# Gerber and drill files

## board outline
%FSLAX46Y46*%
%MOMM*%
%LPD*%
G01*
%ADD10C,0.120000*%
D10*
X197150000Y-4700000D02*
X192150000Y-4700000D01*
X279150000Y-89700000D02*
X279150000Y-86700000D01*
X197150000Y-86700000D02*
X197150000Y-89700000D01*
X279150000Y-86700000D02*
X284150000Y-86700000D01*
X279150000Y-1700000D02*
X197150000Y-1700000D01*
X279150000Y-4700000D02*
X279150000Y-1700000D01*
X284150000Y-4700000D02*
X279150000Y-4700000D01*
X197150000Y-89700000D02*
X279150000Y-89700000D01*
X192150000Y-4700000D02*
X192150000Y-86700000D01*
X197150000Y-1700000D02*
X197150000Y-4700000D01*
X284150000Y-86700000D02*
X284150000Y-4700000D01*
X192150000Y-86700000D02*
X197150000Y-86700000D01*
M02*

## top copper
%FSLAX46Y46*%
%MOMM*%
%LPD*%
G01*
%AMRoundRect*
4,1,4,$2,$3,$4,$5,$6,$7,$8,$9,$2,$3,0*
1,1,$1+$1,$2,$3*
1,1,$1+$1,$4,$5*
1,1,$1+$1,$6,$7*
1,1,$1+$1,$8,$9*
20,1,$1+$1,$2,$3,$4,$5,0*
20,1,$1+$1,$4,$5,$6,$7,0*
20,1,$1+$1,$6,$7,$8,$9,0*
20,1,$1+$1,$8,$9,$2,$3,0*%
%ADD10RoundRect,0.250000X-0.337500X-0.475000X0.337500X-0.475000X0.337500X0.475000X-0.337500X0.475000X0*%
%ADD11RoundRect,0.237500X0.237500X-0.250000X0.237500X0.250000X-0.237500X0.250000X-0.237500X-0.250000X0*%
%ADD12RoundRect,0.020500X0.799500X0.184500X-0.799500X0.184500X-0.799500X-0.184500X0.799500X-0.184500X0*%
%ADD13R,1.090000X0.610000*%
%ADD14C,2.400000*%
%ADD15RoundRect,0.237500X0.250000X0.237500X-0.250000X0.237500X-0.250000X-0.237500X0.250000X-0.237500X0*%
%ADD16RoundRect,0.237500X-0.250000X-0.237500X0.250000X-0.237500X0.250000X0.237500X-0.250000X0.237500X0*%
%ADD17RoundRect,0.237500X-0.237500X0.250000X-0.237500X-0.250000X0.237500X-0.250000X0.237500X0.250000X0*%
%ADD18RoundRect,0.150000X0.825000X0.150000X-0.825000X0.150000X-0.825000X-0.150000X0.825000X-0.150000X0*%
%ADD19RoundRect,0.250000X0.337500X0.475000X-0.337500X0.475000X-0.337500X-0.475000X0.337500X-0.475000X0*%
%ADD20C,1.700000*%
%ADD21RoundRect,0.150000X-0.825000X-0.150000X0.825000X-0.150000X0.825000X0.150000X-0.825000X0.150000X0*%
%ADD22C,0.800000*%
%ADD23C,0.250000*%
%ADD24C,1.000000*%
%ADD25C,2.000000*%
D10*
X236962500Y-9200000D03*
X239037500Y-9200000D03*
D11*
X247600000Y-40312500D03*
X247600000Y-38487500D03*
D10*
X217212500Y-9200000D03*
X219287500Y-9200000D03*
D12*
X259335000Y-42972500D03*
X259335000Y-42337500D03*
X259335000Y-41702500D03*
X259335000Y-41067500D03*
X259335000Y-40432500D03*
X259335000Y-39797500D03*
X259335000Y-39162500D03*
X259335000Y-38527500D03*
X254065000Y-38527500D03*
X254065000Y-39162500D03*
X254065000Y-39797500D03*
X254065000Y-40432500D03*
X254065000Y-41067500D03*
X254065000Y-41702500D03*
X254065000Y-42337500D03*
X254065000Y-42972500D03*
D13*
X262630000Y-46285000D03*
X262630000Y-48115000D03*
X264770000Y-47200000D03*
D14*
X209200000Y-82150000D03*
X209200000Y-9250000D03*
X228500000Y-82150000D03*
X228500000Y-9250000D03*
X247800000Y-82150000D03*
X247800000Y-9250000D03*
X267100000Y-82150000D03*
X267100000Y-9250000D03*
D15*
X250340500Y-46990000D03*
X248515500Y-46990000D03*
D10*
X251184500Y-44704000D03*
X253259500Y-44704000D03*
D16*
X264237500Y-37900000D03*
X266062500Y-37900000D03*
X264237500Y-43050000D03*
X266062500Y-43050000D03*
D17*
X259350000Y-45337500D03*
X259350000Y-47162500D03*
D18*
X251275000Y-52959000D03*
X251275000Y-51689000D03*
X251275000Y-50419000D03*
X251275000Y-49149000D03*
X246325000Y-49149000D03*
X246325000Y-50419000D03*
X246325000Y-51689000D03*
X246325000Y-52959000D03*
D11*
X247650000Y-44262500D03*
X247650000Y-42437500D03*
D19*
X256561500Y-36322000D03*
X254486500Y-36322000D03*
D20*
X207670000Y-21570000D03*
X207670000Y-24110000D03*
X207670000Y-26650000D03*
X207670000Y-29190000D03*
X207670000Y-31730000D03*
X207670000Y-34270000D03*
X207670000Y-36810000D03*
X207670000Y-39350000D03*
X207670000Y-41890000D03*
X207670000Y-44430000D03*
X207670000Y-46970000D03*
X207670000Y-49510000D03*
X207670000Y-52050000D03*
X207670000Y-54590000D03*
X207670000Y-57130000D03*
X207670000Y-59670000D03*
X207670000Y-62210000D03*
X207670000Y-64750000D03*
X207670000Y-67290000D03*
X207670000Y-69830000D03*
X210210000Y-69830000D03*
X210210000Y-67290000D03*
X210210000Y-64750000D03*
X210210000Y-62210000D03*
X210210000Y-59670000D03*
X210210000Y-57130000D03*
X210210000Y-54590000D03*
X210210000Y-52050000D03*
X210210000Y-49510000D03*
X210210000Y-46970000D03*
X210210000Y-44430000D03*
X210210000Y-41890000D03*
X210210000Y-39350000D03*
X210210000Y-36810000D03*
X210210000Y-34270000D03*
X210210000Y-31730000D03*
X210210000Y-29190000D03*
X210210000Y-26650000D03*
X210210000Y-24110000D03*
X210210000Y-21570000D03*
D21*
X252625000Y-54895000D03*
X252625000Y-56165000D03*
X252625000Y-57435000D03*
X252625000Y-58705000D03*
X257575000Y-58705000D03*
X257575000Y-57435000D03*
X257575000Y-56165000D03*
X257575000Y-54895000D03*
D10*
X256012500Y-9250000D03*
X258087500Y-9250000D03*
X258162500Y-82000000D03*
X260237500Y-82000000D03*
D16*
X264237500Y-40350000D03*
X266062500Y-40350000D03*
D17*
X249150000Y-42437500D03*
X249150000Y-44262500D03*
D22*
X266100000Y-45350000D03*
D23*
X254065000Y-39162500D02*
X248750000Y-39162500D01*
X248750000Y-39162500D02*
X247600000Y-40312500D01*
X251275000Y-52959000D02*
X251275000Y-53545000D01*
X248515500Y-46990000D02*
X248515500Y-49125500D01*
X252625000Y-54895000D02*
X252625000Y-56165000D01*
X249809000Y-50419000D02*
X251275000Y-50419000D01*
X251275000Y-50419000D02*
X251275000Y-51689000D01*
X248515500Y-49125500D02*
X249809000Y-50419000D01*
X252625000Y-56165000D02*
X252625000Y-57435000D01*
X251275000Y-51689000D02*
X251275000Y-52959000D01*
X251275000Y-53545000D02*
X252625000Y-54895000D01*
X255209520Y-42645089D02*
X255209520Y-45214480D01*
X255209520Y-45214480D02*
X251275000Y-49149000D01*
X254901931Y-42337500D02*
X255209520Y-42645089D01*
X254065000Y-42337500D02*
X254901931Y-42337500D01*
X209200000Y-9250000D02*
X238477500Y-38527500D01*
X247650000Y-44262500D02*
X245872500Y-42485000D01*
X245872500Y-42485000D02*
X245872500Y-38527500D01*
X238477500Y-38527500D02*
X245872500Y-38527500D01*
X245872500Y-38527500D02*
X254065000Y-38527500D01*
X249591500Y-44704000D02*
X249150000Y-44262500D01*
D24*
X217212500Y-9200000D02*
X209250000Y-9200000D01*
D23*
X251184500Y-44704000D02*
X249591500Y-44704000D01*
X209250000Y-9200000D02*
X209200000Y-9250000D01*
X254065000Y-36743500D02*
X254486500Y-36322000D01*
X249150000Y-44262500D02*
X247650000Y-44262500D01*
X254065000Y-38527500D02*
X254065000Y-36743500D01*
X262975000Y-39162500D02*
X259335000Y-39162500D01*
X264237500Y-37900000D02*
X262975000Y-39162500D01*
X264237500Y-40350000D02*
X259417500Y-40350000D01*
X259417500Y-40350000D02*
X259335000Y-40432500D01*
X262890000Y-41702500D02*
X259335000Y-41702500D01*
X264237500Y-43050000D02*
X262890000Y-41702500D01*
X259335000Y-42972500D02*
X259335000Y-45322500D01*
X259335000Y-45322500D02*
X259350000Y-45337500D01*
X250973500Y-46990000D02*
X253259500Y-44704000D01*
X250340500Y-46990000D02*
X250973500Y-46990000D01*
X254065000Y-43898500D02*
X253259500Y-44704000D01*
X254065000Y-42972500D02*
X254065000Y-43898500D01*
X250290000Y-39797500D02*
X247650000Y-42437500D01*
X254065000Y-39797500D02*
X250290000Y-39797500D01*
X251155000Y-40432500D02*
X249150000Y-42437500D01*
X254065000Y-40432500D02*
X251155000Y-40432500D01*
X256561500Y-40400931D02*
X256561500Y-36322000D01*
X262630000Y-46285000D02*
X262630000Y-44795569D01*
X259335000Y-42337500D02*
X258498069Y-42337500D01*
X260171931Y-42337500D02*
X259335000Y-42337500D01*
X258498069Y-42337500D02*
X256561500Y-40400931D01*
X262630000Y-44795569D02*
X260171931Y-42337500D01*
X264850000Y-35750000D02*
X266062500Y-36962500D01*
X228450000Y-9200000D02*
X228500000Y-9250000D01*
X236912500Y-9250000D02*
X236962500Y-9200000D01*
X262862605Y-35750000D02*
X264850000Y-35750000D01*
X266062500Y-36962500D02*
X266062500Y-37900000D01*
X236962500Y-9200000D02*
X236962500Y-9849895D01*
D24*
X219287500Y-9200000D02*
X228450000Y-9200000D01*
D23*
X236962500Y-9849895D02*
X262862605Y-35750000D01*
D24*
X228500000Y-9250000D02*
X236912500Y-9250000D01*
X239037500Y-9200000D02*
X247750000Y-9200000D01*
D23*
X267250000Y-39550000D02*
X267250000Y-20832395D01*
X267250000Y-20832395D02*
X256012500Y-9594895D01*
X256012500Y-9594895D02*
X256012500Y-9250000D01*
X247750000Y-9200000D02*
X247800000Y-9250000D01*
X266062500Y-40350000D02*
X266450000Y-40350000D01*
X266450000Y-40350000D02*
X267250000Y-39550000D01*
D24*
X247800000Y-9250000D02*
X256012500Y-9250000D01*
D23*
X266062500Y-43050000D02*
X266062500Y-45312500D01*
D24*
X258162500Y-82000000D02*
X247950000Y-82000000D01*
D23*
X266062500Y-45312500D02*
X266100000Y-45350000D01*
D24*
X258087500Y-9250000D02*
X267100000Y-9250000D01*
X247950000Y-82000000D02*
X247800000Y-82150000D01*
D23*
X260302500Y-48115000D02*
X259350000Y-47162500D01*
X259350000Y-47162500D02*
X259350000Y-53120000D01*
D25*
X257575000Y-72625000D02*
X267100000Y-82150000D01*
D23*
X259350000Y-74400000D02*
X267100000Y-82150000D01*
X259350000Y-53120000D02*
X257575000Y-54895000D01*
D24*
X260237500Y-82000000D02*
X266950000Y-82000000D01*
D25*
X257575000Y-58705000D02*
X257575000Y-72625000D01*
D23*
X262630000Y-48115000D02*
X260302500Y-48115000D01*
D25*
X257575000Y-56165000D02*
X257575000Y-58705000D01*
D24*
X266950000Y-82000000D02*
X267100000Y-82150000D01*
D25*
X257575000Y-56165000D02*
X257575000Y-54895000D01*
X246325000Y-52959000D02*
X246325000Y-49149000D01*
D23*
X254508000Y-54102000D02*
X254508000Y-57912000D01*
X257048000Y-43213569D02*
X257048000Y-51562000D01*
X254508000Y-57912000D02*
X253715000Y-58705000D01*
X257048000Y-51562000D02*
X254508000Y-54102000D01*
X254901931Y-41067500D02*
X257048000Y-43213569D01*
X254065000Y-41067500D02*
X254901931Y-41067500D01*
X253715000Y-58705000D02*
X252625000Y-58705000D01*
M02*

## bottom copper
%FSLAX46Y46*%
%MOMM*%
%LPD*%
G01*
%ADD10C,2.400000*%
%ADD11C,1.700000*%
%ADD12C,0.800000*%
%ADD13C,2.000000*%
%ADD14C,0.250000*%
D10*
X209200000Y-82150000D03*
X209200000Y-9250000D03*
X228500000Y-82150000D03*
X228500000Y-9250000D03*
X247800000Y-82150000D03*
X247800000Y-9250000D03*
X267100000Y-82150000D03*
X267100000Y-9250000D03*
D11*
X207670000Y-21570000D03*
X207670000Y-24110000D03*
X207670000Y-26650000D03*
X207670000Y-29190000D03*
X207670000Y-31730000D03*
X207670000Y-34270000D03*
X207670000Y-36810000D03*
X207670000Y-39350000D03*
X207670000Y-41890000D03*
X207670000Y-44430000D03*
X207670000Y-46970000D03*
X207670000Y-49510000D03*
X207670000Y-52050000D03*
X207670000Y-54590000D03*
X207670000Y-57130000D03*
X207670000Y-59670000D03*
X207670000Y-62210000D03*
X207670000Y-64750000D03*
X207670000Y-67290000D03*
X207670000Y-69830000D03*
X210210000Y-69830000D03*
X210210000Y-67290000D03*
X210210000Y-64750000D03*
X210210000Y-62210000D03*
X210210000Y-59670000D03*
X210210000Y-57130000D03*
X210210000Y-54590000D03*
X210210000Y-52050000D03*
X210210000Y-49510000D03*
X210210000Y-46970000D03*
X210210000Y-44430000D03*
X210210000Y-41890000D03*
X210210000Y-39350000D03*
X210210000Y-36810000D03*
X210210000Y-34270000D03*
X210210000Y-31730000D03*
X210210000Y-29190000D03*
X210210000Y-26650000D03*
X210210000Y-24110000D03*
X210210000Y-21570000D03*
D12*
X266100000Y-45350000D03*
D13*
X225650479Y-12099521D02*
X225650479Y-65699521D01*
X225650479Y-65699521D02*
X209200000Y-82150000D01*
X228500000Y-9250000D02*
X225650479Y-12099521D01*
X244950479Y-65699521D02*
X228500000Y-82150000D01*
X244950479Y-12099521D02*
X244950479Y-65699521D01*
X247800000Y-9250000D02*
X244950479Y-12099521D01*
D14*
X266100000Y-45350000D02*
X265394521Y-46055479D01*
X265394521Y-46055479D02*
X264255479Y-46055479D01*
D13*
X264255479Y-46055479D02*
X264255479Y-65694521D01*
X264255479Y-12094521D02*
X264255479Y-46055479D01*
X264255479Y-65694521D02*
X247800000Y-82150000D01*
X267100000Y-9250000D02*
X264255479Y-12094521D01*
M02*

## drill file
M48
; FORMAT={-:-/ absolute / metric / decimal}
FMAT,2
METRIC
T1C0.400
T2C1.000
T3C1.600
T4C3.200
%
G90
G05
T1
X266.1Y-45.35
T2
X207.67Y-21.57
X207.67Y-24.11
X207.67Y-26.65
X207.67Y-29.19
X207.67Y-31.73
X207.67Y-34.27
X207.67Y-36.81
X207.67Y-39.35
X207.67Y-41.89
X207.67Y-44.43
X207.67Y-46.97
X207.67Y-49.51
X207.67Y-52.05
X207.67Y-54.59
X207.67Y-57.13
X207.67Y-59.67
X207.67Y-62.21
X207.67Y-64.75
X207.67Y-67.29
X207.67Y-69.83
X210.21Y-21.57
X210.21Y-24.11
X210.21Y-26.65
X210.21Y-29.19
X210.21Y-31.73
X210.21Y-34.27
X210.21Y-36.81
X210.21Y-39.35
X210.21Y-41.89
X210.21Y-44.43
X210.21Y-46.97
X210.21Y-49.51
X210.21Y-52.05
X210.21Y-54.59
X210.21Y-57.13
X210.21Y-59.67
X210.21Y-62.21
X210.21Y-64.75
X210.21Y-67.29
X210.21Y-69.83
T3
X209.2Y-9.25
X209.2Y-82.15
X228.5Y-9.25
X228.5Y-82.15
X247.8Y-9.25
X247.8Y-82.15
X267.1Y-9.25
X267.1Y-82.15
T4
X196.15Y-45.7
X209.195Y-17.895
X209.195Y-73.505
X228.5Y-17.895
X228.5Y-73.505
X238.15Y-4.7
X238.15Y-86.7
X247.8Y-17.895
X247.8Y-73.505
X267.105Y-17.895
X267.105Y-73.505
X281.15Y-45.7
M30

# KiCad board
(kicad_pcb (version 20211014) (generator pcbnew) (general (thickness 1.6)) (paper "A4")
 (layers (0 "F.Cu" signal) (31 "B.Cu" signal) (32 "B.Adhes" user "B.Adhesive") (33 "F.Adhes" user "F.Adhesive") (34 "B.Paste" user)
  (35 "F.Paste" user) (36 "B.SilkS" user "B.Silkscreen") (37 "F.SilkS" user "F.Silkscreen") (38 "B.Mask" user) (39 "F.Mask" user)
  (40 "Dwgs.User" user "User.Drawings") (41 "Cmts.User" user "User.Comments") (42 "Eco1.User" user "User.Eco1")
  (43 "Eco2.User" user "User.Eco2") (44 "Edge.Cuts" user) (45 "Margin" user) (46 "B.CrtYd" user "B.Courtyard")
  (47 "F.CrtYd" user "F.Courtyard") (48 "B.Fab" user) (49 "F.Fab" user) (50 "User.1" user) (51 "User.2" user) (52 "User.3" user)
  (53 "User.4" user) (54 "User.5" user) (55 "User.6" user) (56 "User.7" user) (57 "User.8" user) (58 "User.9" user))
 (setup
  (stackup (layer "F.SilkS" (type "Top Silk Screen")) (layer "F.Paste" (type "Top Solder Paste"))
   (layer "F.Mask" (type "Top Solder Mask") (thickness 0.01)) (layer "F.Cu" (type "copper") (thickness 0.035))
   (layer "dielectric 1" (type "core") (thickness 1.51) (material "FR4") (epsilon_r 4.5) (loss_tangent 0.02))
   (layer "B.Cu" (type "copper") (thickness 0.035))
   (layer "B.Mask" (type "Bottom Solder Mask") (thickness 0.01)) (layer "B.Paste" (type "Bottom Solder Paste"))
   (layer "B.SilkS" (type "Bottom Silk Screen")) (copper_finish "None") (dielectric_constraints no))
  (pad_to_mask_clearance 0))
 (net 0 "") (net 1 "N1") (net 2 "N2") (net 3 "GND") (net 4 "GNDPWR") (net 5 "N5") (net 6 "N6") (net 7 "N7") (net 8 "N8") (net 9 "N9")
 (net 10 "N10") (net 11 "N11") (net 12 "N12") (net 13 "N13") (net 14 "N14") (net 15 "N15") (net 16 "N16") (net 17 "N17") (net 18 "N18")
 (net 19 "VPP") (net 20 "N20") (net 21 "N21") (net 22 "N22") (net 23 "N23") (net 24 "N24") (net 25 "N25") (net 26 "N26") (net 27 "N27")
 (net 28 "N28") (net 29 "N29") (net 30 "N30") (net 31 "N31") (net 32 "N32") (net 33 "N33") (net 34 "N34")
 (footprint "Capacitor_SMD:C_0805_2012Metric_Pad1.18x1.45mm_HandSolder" (layer "F.Cu") (at 238 9.2)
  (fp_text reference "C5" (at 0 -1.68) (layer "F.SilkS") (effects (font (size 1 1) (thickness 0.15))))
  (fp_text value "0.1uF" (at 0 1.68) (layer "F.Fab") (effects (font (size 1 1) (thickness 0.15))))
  (pad "1" smd roundrect (at -1.0375 0) (size 1.175 1.45) (layers "F.Cu" "F.Paste" "F.Mask") (roundrect_rratio 0.212766) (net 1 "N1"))
  (pad "2" smd roundrect (at 1.0375 0) (size 1.175 1.45) (layers "F.Cu" "F.Paste" "F.Mask") (roundrect_rratio 0.212766) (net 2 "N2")))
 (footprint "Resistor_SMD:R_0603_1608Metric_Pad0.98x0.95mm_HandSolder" (layer "F.Cu") (at 247.6 39.4 90)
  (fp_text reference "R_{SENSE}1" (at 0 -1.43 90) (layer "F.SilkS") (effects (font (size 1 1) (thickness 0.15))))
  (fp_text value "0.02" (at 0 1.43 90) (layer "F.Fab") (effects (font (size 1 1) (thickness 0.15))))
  (pad "1" smd roundrect (at -0.9125 0 90) (size 0.975 0.95) (layers "F.Cu" "F.Paste" "F.Mask") (roundrect_rratio 0.25) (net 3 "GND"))
  (pad "2" smd roundrect (at 0.9125 0 90) (size 0.975 0.95) (layers "F.Cu" "F.Paste" "F.Mask") (roundrect_rratio 0.25) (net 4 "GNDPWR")))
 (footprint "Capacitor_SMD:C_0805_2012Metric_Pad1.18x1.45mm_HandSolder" (layer "F.Cu") (at 218.25 9.2)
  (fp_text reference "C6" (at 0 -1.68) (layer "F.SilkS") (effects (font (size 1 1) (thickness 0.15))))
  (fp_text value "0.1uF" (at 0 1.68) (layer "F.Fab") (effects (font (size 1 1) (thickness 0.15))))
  (pad "1" smd roundrect (at -1.0375 0) (size 1.175 1.45) (layers "F.Cu" "F.Paste" "F.Mask") (roundrect_rratio 0.212766) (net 4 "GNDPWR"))
  (pad "2" smd roundrect (at 1.0375 0) (size 1.175 1.45) (layers "F.Cu" "F.Paste" "F.Mask") (roundrect_rratio 0.212766) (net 1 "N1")))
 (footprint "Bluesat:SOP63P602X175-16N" (layer "F.Cu") (at 256.7 40.75 180)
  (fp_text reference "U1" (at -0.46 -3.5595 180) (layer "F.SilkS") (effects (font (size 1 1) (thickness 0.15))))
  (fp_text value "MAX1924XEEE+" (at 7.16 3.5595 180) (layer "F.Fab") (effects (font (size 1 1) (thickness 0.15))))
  (pad "1" smd roundrect locked (at -2.635 -2.2225 180) (size 1.64 0.41) (layers "F.Cu" "F.Paste" "F.Mask") (roundrect_rratio 0.05)
   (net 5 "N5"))
  (pad "2" smd roundrect locked (at -2.635 -1.5875 180) (size 1.64 0.41) (layers "F.Cu" "F.Paste" "F.Mask") (roundrect_rratio 0.05)
   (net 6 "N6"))
  (pad "3" smd roundrect locked (at -2.635 -0.9525 180) (size 1.64 0.41) (layers "F.Cu" "F.Paste" "F.Mask") (roundrect_rratio 0.05)
   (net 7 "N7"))
  (pad "4" smd roundrect locked (at -2.635 -0.3175 180) (size 1.64 0.41) (layers "F.Cu" "F.Paste" "F.Mask") (roundrect_rratio 0.05))
  (pad "5" smd roundrect locked (at -2.635 0.3175 180) (size 1.64 0.41) (layers "F.Cu" "F.Paste" "F.Mask") (roundrect_rratio 0.05)
   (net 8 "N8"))
  (pad "6" smd roundrect locked (at -2.635 0.9525 180) (size 1.64 0.41) (layers "F.Cu" "F.Paste" "F.Mask") (roundrect_rratio 0.05))
  (pad "7" smd roundrect locked (at -2.635 1.5875 180) (size 1.64 0.41) (layers "F.Cu" "F.Paste" "F.Mask") (roundrect_rratio 0.05)
   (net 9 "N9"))
  (pad "8" smd roundrect locked (at -2.635 2.2225 180) (size 1.64 0.41) (layers "F.Cu" "F.Paste" "F.Mask") (roundrect_rratio 0.05))
  (pad "9" smd roundrect locked (at 2.635 2.2225 180) (size 1.64 0.41) (layers "F.Cu" "F.Paste" "F.Mask") (roundrect_rratio 0.05)
   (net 4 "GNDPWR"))
  (pad "10" smd roundrect locked (at 2.635 1.5875 180) (size 1.64 0.41) (layers "F.Cu" "F.Paste" "F.Mask") (roundrect_rratio 0.05)
   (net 3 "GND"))
  (pad "11" smd roundrect locked (at 2.635 0.9525 180) (size 1.64 0.41) (layers "F.Cu" "F.Paste" "F.Mask") (roundrect_rratio 0.05)
   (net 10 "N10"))
  (pad "12" smd roundrect locked (at 2.635 0.3175 180) (size 1.64 0.41) (layers "F.Cu" "F.Paste" "F.Mask") (roundrect_rratio 0.05)
   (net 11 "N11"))
  (pad "13" smd roundrect locked (at 2.635 -0.3175 180) (size 1.64 0.41) (layers "F.Cu" "F.Paste" "F.Mask") (roundrect_rratio 0.05)
   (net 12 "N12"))
  (pad "14" smd roundrect locked (at 2.635 -0.9525 180) (size 1.64 0.41) (layers "F.Cu" "F.Paste" "F.Mask") (roundrect_rratio 0.05)
   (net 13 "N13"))
  (pad "15" smd roundrect locked (at 2.635 -1.5875 180) (size 1.64 0.41) (layers "F.Cu" "F.Paste" "F.Mask") (roundrect_rratio 0.05)
   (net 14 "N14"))
  (pad "16" smd roundrect locked (at 2.635 -2.2225 180) (size 1.64 0.41) (layers "F.Cu" "F.Paste" "F.Mask") (roundrect_rratio 0.05)
   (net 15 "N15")))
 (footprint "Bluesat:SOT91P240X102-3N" (layer "F.Cu") (at 263.7 47.2 -90)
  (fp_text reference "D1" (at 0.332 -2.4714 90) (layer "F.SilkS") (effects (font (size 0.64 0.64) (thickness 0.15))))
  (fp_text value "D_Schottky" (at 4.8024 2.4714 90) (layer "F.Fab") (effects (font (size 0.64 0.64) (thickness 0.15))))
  (pad "1" smd rect locked (at -0.915 1.07 270) (size 0.61 1.09) (layers "F.Cu" "F.Paste" "F.Mask") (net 6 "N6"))
  (pad "2" smd rect locked (at 0.915 1.07 270) (size 0.61 1.09) (layers "F.Cu" "F.Paste" "F.Mask") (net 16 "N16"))
  (pad "3" smd rect locked (at 0 -1.07 270) (size 0.61 1.09) (layers "F.Cu" "F.Paste" "F.Mask")))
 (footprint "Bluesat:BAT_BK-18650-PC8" (layer "F.Cu") (at 238.15 45.7 90)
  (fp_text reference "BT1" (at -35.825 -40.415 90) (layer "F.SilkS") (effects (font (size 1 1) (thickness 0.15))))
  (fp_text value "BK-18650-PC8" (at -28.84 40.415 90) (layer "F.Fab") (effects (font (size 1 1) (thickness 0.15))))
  (pad "" np_thru_hole circle locked (at 27.805 28.955 90) (size 3.2 3.2) (drill 3.2) (layers *.Cu *.Mask))
  (pad "" np_thru_hole circle locked (at -27.805 -9.65 90) (size 3.2 3.2) (drill 3.2) (layers *.Cu *.Mask))
  (pad "" np_thru_hole circle locked (at -27.805 9.65 90) (size 3.2 3.2) (drill 3.2) (layers *.Cu *.Mask))
  (pad "" np_thru_hole circle locked (at 27.805 -9.65 90) (size 3.2 3.2) (drill 3.2) (layers *.Cu *.Mask))
  (pad "" np_thru_hole circle locked (at 27.805 -28.955 90) (size 3.2 3.2) (drill 3.2) (layers *.Cu *.Mask))
  (pad "" np_thru_hole circle locked (at 27.805 9.65 90) (size 3.2 3.2) (drill 3.2) (layers *.Cu *.Mask))
  (pad "" np_thru_hole circle locked (at -27.805 28.955 90) (size 3.2 3.2) (drill 3.2) (layers *.Cu *.Mask))
  (pad "" np_thru_hole circle locked (at -27.805 -28.955 90) (size 3.2 3.2) (drill 3.2) (layers *.Cu *.Mask))
  (pad "1+" thru_hole circle locked (at -36.45 -28.95 90) (size 2.4 2.4) (drill 1.6) (layers *.Cu *.Mask) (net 1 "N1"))
  (pad "1-" thru_hole circle locked (at 36.45 -28.95 90) (size 2.4 2.4) (drill 1.6) (layers *.Cu *.Mask) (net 4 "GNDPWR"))
  (pad "2+" thru_hole circle locked (at -36.45 -9.65 90) (size 2.4 2.4) (drill 1.6) (layers *.Cu *.Mask) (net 2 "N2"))
  (pad "2-" thru_hole circle locked (at 36.45 -9.65 90) (size 2.4 2.4) (drill 1.6) (layers *.Cu *.Mask) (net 1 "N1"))
  (pad "3+" thru_hole circle locked (at -36.45 9.65 90) (size 2.4 2.4) (drill 1.6) (layers *.Cu *.Mask) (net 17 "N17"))
  (pad "3-" thru_hole circle locked (at 36.45 9.65 90) (size 2.4 2.4) (drill 1.6) (layers *.Cu *.Mask) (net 2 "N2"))
  (pad "4+" thru_hole circle locked (at -36.45 28.95 90) (size 2.4 2.4) (drill 1.6) (layers *.Cu *.Mask) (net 16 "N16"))
  (pad "4-" thru_hole circle locked (at 36.45 28.95 90) (size 2.4 2.4) (drill 1.6) (layers *.Cu *.Mask) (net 17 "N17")))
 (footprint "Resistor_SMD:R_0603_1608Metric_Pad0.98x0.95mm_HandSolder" (layer "F.Cu") (at 249.428 46.99 180)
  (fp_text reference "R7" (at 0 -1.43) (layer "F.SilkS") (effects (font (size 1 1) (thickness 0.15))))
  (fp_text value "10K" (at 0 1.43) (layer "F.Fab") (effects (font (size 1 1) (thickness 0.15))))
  (pad "1" smd roundrect (at -0.9125 0 180) (size 0.975 0.95) (layers "F.Cu" "F.Paste" "F.Mask") (roundrect_rratio 0.25) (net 15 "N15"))
  (pad "2" smd roundrect (at 0.9125 0 180) (size 0.975 0.95) (layers "F.Cu" "F.Paste" "F.Mask") (roundrect_rratio 0.25) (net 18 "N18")))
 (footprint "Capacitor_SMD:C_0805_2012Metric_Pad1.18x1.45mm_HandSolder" (layer "F.Cu") (at 252.222 44.704)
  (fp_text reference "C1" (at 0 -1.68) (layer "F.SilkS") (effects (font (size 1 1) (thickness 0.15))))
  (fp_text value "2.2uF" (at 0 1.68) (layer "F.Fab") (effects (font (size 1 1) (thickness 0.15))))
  (pad "1" smd roundrect (at -1.0375 0) (size 1.175 1.45) (layers "F.Cu" "F.Paste" "F.Mask") (roundrect_rratio 0.212766) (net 4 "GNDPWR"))
  (pad "2" smd roundrect (at 1.0375 0) (size 1.175 1.45) (layers "F.Cu" "F.Paste" "F.Mask") (roundrect_rratio 0.212766) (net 15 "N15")))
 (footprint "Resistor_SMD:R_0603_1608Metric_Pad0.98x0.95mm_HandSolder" (layer "F.Cu") (at 265.15 37.9)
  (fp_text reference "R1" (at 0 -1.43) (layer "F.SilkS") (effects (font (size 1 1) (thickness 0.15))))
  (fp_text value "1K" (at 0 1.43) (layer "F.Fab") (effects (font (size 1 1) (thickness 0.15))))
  (pad "1" smd roundrect (at -0.9125 0) (size 0.975 0.95) (layers "F.Cu" "F.Paste" "F.Mask") (roundrect_rratio 0.25) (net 9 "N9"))
  (pad "2" smd roundrect (at 0.9125 0) (size 0.975 0.95) (layers "F.Cu" "F.Paste" "F.Mask") (roundrect_rratio 0.25) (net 1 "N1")))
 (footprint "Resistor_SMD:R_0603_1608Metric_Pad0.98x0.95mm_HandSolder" (layer "F.Cu") (at 265.15 43.05)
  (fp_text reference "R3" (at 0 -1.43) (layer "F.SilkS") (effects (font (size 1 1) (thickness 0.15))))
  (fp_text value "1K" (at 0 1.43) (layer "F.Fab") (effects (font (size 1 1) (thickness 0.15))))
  (pad "1" smd roundrect (at -0.9125 0) (size 0.975 0.95) (layers "F.Cu" "F.Paste" "F.Mask") (roundrect_rratio 0.25) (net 7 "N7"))
  (pad "2" smd roundrect (at 0.9125 0) (size 0.975 0.95) (layers "F.Cu" "F.Paste" "F.Mask") (roundrect_rratio 0.25) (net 17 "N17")))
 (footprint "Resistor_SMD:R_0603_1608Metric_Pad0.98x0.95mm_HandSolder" (layer "F.Cu") (at 259.35 46.25 -90)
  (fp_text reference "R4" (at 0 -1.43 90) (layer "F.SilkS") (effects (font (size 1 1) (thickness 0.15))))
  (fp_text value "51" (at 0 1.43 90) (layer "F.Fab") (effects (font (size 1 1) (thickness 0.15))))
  (pad "1" smd roundrect (at -0.9125 0 270) (size 0.975 0.95) (layers "F.Cu" "F.Paste" "F.Mask") (roundrect_rratio 0.25) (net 5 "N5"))
  (pad "2" smd roundrect (at 0.9125 0 270) (size 0.975 0.95) (layers "F.Cu" "F.Paste" "F.Mask") (roundrect_rratio 0.25) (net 16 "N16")))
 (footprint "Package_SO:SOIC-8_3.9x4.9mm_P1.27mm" (layer "F.Cu") (at 248.8 51.054 180)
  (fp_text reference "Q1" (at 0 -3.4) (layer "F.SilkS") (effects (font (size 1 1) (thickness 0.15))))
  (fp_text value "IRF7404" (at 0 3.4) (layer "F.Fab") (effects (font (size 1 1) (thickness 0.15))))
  (pad "1" smd roundrect (at -2.475 -1.905 180) (size 1.95 0.6) (layers "F.Cu" "F.Paste" "F.Mask") (roundrect_rratio 0.25) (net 18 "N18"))
  (pad "2" smd roundrect (at -2.475 -0.635 180) (size 1.95 0.6) (layers "F.Cu" "F.Paste" "F.Mask") (roundrect_rratio 0.25) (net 18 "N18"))
  (pad "3" smd roundrect (at -2.475 0.635 180) (size 1.95 0.6) (layers "F.Cu" "F.Paste" "F.Mask") (roundrect_rratio 0.25) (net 18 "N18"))
  (pad "4" smd roundrect (at -2.475 1.905 180) (size 1.95 0.6) (layers "F.Cu" "F.Paste" "F.Mask") (roundrect_rratio 0.25) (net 14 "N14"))
  (pad "5" smd roundrect (at 2.475 1.905 180) (size 1.95 0.6) (layers "F.Cu" "F.Paste" "F.Mask") (roundrect_rratio 0.25) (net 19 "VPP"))
  (pad "6" smd roundrect (at 2.475 0.635 180) (size 1.95 0.6) (layers "F.Cu" "F.Paste" "F.Mask") (roundrect_rratio 0.25) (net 19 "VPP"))
  (pad "7" smd roundrect (at 2.475 -0.635 180) (size 1.95 0.6) (layers "F.Cu" "F.Paste" "F.Mask") (roundrect_rratio 0.25) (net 19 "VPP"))
  (pad "8" smd roundrect (at 2.475 -1.905 180) (size 1.95 0.6) (layers "F.Cu" "F.Paste" "F.Mask") (roundrect_rratio 0.25) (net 19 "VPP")))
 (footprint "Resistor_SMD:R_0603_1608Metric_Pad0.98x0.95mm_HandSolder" (layer "F.Cu") (at 247.65 43.35 90)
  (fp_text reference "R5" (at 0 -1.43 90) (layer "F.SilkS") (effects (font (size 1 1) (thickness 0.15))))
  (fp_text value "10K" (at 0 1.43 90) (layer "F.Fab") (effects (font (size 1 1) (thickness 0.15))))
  (pad "1" smd roundrect (at -0.9125 0 90) (size 0.975 0.95) (layers "F.Cu" "F.Paste" "F.Mask") (roundrect_rratio 0.25) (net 4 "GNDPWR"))
  (pad "2" smd roundrect (at 0.9125 0 90) (size 0.975 0.95) (layers "F.Cu" "F.Paste" "F.Mask") (roundrect_rratio 0.25) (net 10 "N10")))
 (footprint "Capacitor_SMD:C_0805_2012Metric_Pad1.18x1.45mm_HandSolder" (layer "F.Cu") (at 255.524 36.322 180)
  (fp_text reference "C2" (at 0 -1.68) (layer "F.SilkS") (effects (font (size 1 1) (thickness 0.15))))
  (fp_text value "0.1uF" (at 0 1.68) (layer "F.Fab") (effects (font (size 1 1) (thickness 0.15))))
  (pad "1" smd roundrect (at -1.0375 0 180) (size 1.175 1.45) (layers "F.Cu" "F.Paste" "F.Mask") (roundrect_rratio 0.212766) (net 6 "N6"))
  (pad "2" smd roundrect (at 1.0375 0 180) (size 1.175 1.45) (layers "F.Cu" "F.Paste" "F.Mask") (roundrect_rratio 0.212766) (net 4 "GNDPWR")))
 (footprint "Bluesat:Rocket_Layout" (layer "F.Cu") (at 238.15 45.7)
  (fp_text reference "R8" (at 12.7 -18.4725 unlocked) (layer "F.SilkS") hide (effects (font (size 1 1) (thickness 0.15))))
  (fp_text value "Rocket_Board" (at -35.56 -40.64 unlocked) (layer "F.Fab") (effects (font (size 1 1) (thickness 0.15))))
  (fp_line (start -41 -41) (end -46 -41) (layer "Edge.Cuts") (width 0.12))
  (fp_line (start 41 44) (end 41 41) (layer "Edge.Cuts") (width 0.12))
  (fp_line (start -41 41) (end -41 44) (layer "Edge.Cuts") (width 0.12))
  (fp_line (start 41 41) (end 46 41) (layer "Edge.Cuts") (width 0.12))
  (fp_line (start 41 -44) (end -41 -44) (layer "Edge.Cuts") (width 0.12))
  (fp_line (start 41 -41) (end 41 -44) (layer "Edge.Cuts") (width 0.12))
  (fp_line (start 46 -41) (end 41 -41) (layer "Edge.Cuts") (width 0.12))
  (fp_line (start -41 44) (end 41 44) (layer "Edge.Cuts") (width 0.12))
  (fp_line (start -46 -41) (end -46 41) (layer "Edge.Cuts") (width 0.12))
  (fp_line (start -41 -44) (end -41 -41) (layer "Edge.Cuts") (width 0.12))
  (fp_line (start 46 41) (end 46 -41) (layer "Edge.Cuts") (width 0.12))
  (fp_line (start -46 41) (end -41 41) (layer "Edge.Cuts") (width 0.12))
  (pad "" np_thru_hole circle locked (at -42 0) (size 2 2) (drill 3.2) (layers *.Mask))
  (pad "" np_thru_hole circle locked (at 0 -41) (size 2 2) (drill 3.2) (layers *.Mask))
  (pad "" np_thru_hole circle locked (at 0 41) (size 2 2) (drill 3.2) (layers *.Mask))
  (pad "" np_thru_hole circle locked (at 43 0) (size 2 2) (drill 3.2) (layers *.Mask))
  (pad "1" thru_hole circle locked (at -30.48 -24.13) (size 1.7 1.7) (drill 1) (layers *.Cu *.Mask) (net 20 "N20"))
  (pad "2" thru_hole circle locked (at -30.48 -21.59) (size 1.7 1.7) (drill 1) (layers *.Cu *.Mask) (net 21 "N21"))
  (pad "3" thru_hole circle locked (at -30.48 -19.05) (size 1.7 1.7) (drill 1) (layers *.Cu *.Mask) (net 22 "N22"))
  (pad "4" thru_hole circle locked (at -30.48 -16.51) (size 1.7 1.7) (drill 1) (layers *.Cu *.Mask) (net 21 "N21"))
  (pad "5" thru_hole circle locked (at -30.48 -13.97) (size 1.7 1.7) (drill 1) (layers *.Cu *.Mask) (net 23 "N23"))
  (pad "6" thru_hole circle locked (at -30.48 -11.43) (size 1.7 1.7) (drill 1) (layers *.Cu *.Mask) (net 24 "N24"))
  (pad "7" thru_hole circle locked (at -30.48 -8.89) (size 1.7 1.7) (drill 1) (layers *.Cu *.Mask) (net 21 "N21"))
  (pad "8" thru_hole circle locked (at -30.48 -6.35) (size 1.7 1.7) (drill 1) (layers *.Cu *.Mask) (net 20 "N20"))
  (pad "9" thru_hole circle locked (at -30.48 -3.81) (size 1.7 1.7) (drill 1) (layers *.Cu *.Mask) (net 21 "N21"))
  (pad "10" thru_hole circle locked (at -30.48 -1.27) (size 1.7 1.7) (drill 1) (layers *.Cu *.Mask) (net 22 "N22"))
  (pad "11" thru_hole circle locked (at -30.48 1.27) (size 1.7 1.7) (drill 1) (layers *.Cu *.Mask) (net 21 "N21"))
  (pad "12" thru_hole circle locked (at -30.48 3.81) (size 1.7 1.7) (drill 1) (layers *.Cu *.Mask) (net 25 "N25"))
  (pad "13" thru_hole circle locked (at -30.48 6.35) (size 1.7 1.7) (drill 1) (layers *.Cu *.Mask) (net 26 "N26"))
  (pad "14" thru_hole circle locked (at -30.48 8.89) (size 1.7 1.7) (drill 1) (layers *.Cu *.Mask) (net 21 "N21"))
  (pad "15" thru_hole circle locked (at -30.48 11.43) (size 1.7 1.7) (drill 1) (layers *.Cu *.Mask) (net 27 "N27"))
  (pad "16" thru_hole circle locked (at -30.48 13.97) (size 1.7 1.7) (drill 1) (layers *.Cu *.Mask) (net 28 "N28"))
  (pad "17" thru_hole circle locked (at -30.48 16.51) (size 1.7 1.7) (drill 1) (layers *.Cu *.Mask) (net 21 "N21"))
  (pad "18" thru_hole circle locked (at -30.48 19.05) (size 1.7 1.7) (drill 1) (layers *.Cu *.Mask) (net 20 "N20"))
  (pad "19" thru_hole circle locked (at -30.48 21.59) (size 1.7 1.7) (drill 1) (layers *.Cu *.Mask) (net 21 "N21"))
  (pad "20" thru_hole circle locked (at -30.48 24.13) (size 1.7 1.7) (drill 1) (layers *.Cu *.Mask) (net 22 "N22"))
  (pad "21" thru_hole circle locked (at -27.94 24.13) (size 1.7 1.7) (drill 1) (layers *.Cu *.Mask) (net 22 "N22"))
  (pad "22" thru_hole circle locked (at -27.94 21.59) (size 1.7 1.7) (drill 1) (layers *.Cu *.Mask) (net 21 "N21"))
  (pad "23" thru_hole circle locked (at -27.94 19.05) (size 1.7 1.7) (drill 1) (layers *.Cu *.Mask) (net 20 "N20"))
  (pad "24" thru_hole circle locked (at -27.94 16.51) (size 1.7 1.7) (drill 1) (layers *.Cu *.Mask) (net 21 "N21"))
  (pad "25" thru_hole circle locked (at -27.94 13.97) (size 1.7 1.7) (drill 1) (layers *.Cu *.Mask) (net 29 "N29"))
  (pad "26" thru_hole circle locked (at -27.94 11.43) (size 1.7 1.7) (drill 1) (layers *.Cu *.Mask) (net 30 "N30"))
  (pad "27" thru_hole circle locked (at -27.94 8.89) (size 1.7 1.7) (drill 1) (layers *.Cu *.Mask) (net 21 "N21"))
  (pad "28" thru_hole circle locked (at -27.94 6.35) (size 1.7 1.7) (drill 1) (layers *.Cu *.Mask) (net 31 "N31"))
  (pad "29" thru_hole circle locked (at -27.94 3.81) (size 1.7 1.7) (drill 1) (layers *.Cu *.Mask) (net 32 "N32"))
  (pad "30" thru_hole circle locked (at -27.94 1.27) (size 1.7 1.7) (drill 1) (layers *.Cu *.Mask) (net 21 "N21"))
  (pad "31" thru_hole circle locked (at -27.94 -1.27) (size 1.7 1.7) (drill 1) (layers *.Cu *.Mask) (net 22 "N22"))
  (pad "32" thru_hole circle locked (at -27.94 -3.81) (size 1.7 1.7) (drill 1) (layers *.Cu *.Mask) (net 21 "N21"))
  (pad "33" thru_hole circle locked (at -27.94 -6.35) (size 1.7 1.7) (drill 1) (layers *.Cu *.Mask) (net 20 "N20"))
  (pad "34" thru_hole circle locked (at -27.94 -8.89) (size 1.7 1.7) (drill 1) (layers *.Cu *.Mask) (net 21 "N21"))
  (pad "35" thru_hole circle locked (at -27.94 -11.43) (size 1.7 1.7) (drill 1) (layers *.Cu *.Mask) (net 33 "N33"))
  (pad "36" thru_hole circle locked (at -27.94 -13.97) (size 1.7 1.7) (drill 1) (layers *.Cu *.Mask) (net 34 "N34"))
  (pad "37" thru_hole circle locked (at -27.94 -16.51) (size 1.7 1.7) (drill 1) (layers *.Cu *.Mask) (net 21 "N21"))
  (pad "38" thru_hole circle locked (at -27.94 -19.05) (size 1.7 1.7) (drill 1) (layers *.Cu *.Mask) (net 22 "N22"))
  (pad "39" thru_hole circle locked (at -27.94 -21.59) (size 1.7 1.7) (drill 1) (layers *.Cu *.Mask) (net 21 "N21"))
  (pad "40" thru_hole circle locked (at -27.94 -24.13) (size 1.7 1.7) (drill 1) (layers *.Cu *.Mask) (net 20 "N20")))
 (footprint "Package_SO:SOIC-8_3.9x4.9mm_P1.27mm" (layer "F.Cu") (at 255.1 56.8)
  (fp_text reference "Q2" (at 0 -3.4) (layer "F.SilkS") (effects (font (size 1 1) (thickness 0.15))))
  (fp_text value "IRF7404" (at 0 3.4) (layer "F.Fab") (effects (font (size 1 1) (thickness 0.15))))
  (pad "1" smd roundrect (at -2.475 -1.905) (size 1.95 0.6) (layers "F.Cu" "F.Paste" "F.Mask") (roundrect_rratio 0.25) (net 18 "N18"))
  (pad "2" smd roundrect (at -2.475 -0.635) (size 1.95 0.6) (layers "F.Cu" "F.Paste" "F.Mask") (roundrect_rratio 0.25) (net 18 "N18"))
  (pad "3" smd roundrect (at -2.475 0.635) (size 1.95 0.6) (layers "F.Cu" "F.Paste" "F.Mask") (roundrect_rratio 0.25) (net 18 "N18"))
  (pad "4" smd roundrect (at -2.475 1.905) (size 1.95 0.6) (layers "F.Cu" "F.Paste" "F.Mask") (roundrect_rratio 0.25) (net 12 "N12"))
  (pad "5" smd roundrect (at 2.475 1.905) (size 1.95 0.6) (layers "F.Cu" "F.Paste" "F.Mask") (roundrect_rratio 0.25) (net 16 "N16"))
  (pad "6" smd roundrect (at 2.475 0.635) (size 1.95 0.6) (layers "F.Cu" "F.Paste" "F.Mask") (roundrect_rratio 0.25) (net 16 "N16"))
  (pad "7" smd roundrect (at 2.475 -0.635) (size 1.95 0.6) (layers "F.Cu" "F.Paste" "F.Mask") (roundrect_rratio 0.25) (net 16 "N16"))
  (pad "8" smd roundrect (at 2.475 -1.905) (size 1.95 0.6) (layers "F.Cu" "F.Paste" "F.Mask") (roundrect_rratio 0.25) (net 16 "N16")))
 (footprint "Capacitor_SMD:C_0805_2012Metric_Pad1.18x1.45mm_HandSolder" (layer "F.Cu") (at 257.05 9.25)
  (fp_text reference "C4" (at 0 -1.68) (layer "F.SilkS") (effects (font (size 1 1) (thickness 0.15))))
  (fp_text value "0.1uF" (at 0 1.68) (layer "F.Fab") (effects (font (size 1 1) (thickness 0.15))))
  (pad "1" smd roundrect (at -1.0375 0) (size 1.175 1.45) (layers "F.Cu" "F.Paste" "F.Mask") (roundrect_rratio 0.212766) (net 2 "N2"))
  (pad "2" smd roundrect (at 1.0375 0) (size 1.175 1.45) (layers "F.Cu" "F.Paste" "F.Mask") (roundrect_rratio 0.212766) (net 17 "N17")))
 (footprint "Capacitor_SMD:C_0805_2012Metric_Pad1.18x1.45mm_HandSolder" (layer "F.Cu") (at 259.2 82)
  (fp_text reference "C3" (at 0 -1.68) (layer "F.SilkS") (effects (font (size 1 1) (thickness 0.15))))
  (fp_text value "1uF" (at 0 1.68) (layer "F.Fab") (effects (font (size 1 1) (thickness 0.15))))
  (pad "1" smd roundrect (at -1.0375 0) (size 1.175 1.45) (layers "F.Cu" "F.Paste" "F.Mask") (roundrect_rratio 0.212766) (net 17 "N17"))
  (pad "2" smd roundrect (at 1.0375 0) (size 1.175 1.45) (layers "F.Cu" "F.Paste" "F.Mask") (roundrect_rratio 0.212766) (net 16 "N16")))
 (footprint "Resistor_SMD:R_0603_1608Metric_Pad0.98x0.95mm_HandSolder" (layer "F.Cu") (at 265.15 40.35)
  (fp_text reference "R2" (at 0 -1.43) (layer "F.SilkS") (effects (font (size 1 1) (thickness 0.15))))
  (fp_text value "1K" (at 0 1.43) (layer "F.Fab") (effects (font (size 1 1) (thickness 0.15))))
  (pad "1" smd roundrect (at -0.9125 0) (size 0.975 0.95) (layers "F.Cu" "F.Paste" "F.Mask") (roundrect_rratio 0.25) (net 8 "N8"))
  (pad "2" smd roundrect (at 0.9125 0) (size 0.975 0.95) (layers "F.Cu" "F.Paste" "F.Mask") (roundrect_rratio 0.25) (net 2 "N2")))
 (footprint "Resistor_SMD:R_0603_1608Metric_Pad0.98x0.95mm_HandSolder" (layer "F.Cu") (at 249.15 43.35 -90)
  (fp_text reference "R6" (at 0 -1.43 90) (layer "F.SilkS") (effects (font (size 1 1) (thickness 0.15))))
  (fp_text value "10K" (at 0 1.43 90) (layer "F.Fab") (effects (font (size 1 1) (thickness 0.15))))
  (pad "1" smd roundrect (at -0.9125 0 270) (size 0.975 0.95) (layers "F.Cu" "F.Paste" "F.Mask") (roundrect_rratio 0.25) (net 11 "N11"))
  (pad "2" smd roundrect (at 0.9125 0 270) (size 0.975 0.95) (layers "F.Cu" "F.Paste" "F.Mask") (roundrect_rratio 0.25) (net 4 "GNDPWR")))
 (segment (start 254.065 39.1625) (end 248.75 39.1625) (width 0.25) (layer "F.Cu") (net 3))
 (segment (start 248.75 39.1625) (end 247.6 40.3125) (width 0.25) (layer "F.Cu") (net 3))
 (segment (start 251.275 52.959) (end 251.275 53.545) (width 0.25) (layer "F.Cu") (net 18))
 (segment (start 248.5155 46.99) (end 248.5155 49.1255) (width 0.25) (layer "F.Cu") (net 18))
 (segment (start 252.625 54.895) (end 252.625 56.165) (width 0.25) (layer "F.Cu") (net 18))
 (segment (start 249.809 50.419) (end 251.275 50.419) (width 0.25) (layer "F.Cu") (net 18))
 (segment (start 251.275 50.419) (end 251.275 51.689) (width 0.25) (layer "F.Cu") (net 18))
 (segment (start 248.5155 49.1255) (end 249.809 50.419) (width 0.25) (layer "F.Cu") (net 18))
 (segment (start 252.625 56.165) (end 252.625 57.435) (width 0.25) (layer "F.Cu") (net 18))
 (segment (start 251.275 51.689) (end 251.275 52.959) (width 0.25) (layer "F.Cu") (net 18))
 (segment (start 251.275 53.545) (end 252.625 54.895) (width 0.25) (layer "F.Cu") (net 18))
 (segment (start 255.20952 42.645089) (end 255.20952 45.21448) (width 0.25) (layer "F.Cu") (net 14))
 (segment (start 255.20952 45.21448) (end 251.275 49.149) (width 0.25) (layer "F.Cu") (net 14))
 (segment (start 254.901931 42.3375) (end 255.20952 42.645089) (width 0.25) (layer "F.Cu") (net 14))
 (segment (start 254.065 42.3375) (end 254.901931 42.3375) (width 0.25) (layer "F.Cu") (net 14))
 (segment (start 209.2 9.25) (end 238.4775 38.5275) (width 0.25) (layer "F.Cu") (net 4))
 (segment (start 247.65 44.2625) (end 245.8725 42.485) (width 0.25) (layer "F.Cu") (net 4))
 (segment (start 245.8725 42.485) (end 245.8725 38.5275) (width 0.25) (layer "F.Cu") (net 4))
 (segment (start 238.4775 38.5275) (end 245.8725 38.5275) (width 0.25) (layer "F.Cu") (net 4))
 (segment (start 245.8725 38.5275) (end 254.065 38.5275) (width 0.25) (layer "F.Cu") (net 4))
 (segment (start 249.5915 44.704) (end 249.15 44.2625) (width 0.25) (layer "F.Cu") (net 4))
 (segment (start 217.2125 9.2) (end 209.25 9.2) (width 1) (layer "F.Cu") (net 4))
 (segment (start 251.1845 44.704) (end 249.5915 44.704) (width 0.25) (layer "F.Cu") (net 4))
 (segment (start 209.25 9.2) (end 209.2 9.25) (width 0.25) (layer "F.Cu") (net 4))
 (segment (start 254.065 36.7435) (end 254.4865 36.322) (width 0.25) (layer "F.Cu") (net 4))
 (segment (start 249.15 44.2625) (end 247.65 44.2625) (width 0.25) (layer "F.Cu") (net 4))
 (segment (start 254.065 38.5275) (end 254.065 36.7435) (width 0.25) (layer "F.Cu") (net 4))
 (segment (start 262.975 39.1625) (end 259.335 39.1625) (width 0.25) (layer "F.Cu") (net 9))
 (segment (start 264.2375 37.9) (end 262.975 39.1625) (width 0.25) (layer "F.Cu") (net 9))
 (segment (start 264.2375 40.35) (end 259.4175 40.35) (width 0.25) (layer "F.Cu") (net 8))
 (segment (start 259.4175 40.35) (end 259.335 40.4325) (width 0.25) (layer "F.Cu") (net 8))
 (segment (start 262.89 41.7025) (end 259.335 41.7025) (width 0.25) (layer "F.Cu") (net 7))
 (segment (start 264.2375 43.05) (end 262.89 41.7025) (width 0.25) (layer "F.Cu") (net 7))
 (segment (start 259.335 42.9725) (end 259.335 45.3225) (width 0.25) (layer "F.Cu") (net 5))
 (segment (start 259.335 45.3225) (end 259.35 45.3375) (width 0.25) (layer "F.Cu") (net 5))
 (segment (start 250.9735 46.99) (end 253.2595 44.704) (width 0.25) (layer "F.Cu") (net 15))
 (segment (start 250.3405 46.99) (end 250.9735 46.99) (width 0.25) (layer "F.Cu") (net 15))
 (segment (start 254.065 43.8985) (end 253.2595 44.704) (width 0.25) (layer "F.Cu") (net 15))
 (segment (start 254.065 42.9725) (end 254.065 43.8985) (width 0.25) (layer "F.Cu") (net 15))
 (segment (start 250.29 39.7975) (end 247.65 42.4375) (width 0.25) (layer "F.Cu") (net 10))
 (segment (start 254.065 39.7975) (end 250.29 39.7975) (width 0.25) (layer "F.Cu") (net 10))
 (segment (start 251.155 40.4325) (end 249.15 42.4375) (width 0.25) (layer "F.Cu") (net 11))
 (segment (start 254.065 40.4325) (end 251.155 40.4325) (width 0.25) (layer "F.Cu") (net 11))
 (segment (start 256.5615 40.400931) (end 256.5615 36.322) (width 0.25) (layer "F.Cu") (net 6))
 (segment (start 262.63 46.285) (end 262.63 44.795569) (width 0.25) (layer "F.Cu") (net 6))
 (segment (start 259.335 42.3375) (end 258.498069 42.3375) (width 0.25) (layer "F.Cu") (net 6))
 (segment (start 260.171931 42.3375) (end 259.335 42.3375) (width 0.25) (layer "F.Cu") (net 6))
 (segment (start 258.498069 42.3375) (end 256.5615 40.400931) (width 0.25) (layer "F.Cu") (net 6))
 (segment (start 262.63 44.795569) (end 260.171931 42.3375) (width 0.25) (layer "F.Cu") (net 6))
 (segment (start 264.85 35.75) (end 266.0625 36.9625) (width 0.25) (layer "F.Cu") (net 1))
 (segment (start 228.45 9.2) (end 228.5 9.25) (width 0.25) (layer "F.Cu") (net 1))
 (segment (start 236.9125 9.25) (end 236.9625 9.2) (width 0.25) (layer "F.Cu") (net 1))
 (segment (start 262.862605 35.75) (end 264.85 35.75) (width 0.25) (layer "F.Cu") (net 1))
 (segment (start 266.0625 36.9625) (end 266.0625 37.9) (width 0.25) (layer "F.Cu") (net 1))
 (segment (start 236.9625 9.2) (end 236.9625 9.849895) (width 0.25) (layer "F.Cu") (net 1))
 (segment (start 219.2875 9.2) (end 228.45 9.2) (width 1) (layer "F.Cu") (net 1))
 (segment (start 236.9625 9.849895) (end 262.862605 35.75) (width 0.25) (layer "F.Cu") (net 1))
 (segment (start 228.5 9.25) (end 236.9125 9.25) (width 1) (layer "F.Cu") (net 1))
 (segment (start 225.650479 12.099521) (end 225.650479 65.699521) (width 2) (layer "B.Cu") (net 1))
 (segment (start 225.650479 65.699521) (end 209.2 82.15) (width 2) (layer "B.Cu") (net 1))
 (segment (start 228.5 9.25) (end 225.650479 12.099521) (width 2) (layer "B.Cu") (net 1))
 (segment (start 239.0375 9.2) (end 247.75 9.2) (width 1) (layer "F.Cu") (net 2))
 (segment (start 267.25 39.55) (end 267.25 20.832395) (width 0.25) (layer "F.Cu") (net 2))
 (segment (start 267.25 20.832395) (end 256.0125 9.594895) (width 0.25) (layer "F.Cu") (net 2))
 (segment (start 256.0125 9.594895) (end 256.0125 9.25) (width 0.25) (layer "F.Cu") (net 2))
 (segment (start 247.75 9.2) (end 247.8 9.25) (width 0.25) (layer "F.Cu") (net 2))
 (segment (start 266.0625 40.35) (end 266.45 40.35) (width 0.25) (layer "F.Cu") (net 2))
 (segment (start 266.45 40.35) (end 267.25 39.55) (width 0.25) (layer "F.Cu") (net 2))
 (segment (start 247.8 9.25) (end 256.0125 9.25) (width 1) (layer "F.Cu") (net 2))
 (segment (start 244.950479 65.699521) (end 228.5 82.15) (width 2) (layer "B.Cu") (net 2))
 (segment (start 244.950479 12.099521) (end 244.950479 65.699521) (width 2) (layer "B.Cu") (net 2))
 (segment (start 247.8 9.25) (end 244.950479 12.099521) (width 2) (layer "B.Cu") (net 2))
 (segment (start 266.0625 43.05) (end 266.0625 45.3125) (width 0.25) (layer "F.Cu") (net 17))
 (segment (start 258.1625 82) (end 247.95 82) (width 1) (layer "F.Cu") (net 17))
 (segment (start 266.0625 45.3125) (end 266.1 45.35) (width 0.25) (layer "F.Cu") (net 17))
 (segment (start 258.0875 9.25) (end 267.1 9.25) (width 1) (layer "F.Cu") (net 17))
 (segment (start 247.95 82) (end 247.8 82.15) (width 1) (layer "F.Cu") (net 17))
 (via (at 266.1 45.35) (size 0.8) (drill 0.4) (layers "F.Cu" "B.Cu") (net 17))
 (segment (start 266.1 45.35) (end 265.394521 46.055479) (width 0.25) (layer "B.Cu") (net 17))
 (segment (start 265.394521 46.055479) (end 264.255479 46.055479) (width 0.25) (layer "B.Cu") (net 17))
 (segment (start 264.255479 46.055479) (end 264.255479 65.694521) (width 2) (layer "B.Cu") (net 17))
 (segment (start 264.255479 12.094521) (end 264.255479 46.055479) (width 2) (layer "B.Cu") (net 17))
 (segment (start 264.255479 65.694521) (end 247.8 82.15) (width 2) (layer "B.Cu") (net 17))
 (segment (start 267.1 9.25) (end 264.255479 12.094521) (width 2) (layer "B.Cu") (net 17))
 (segment (start 260.3025 48.115) (end 259.35 47.1625) (width 0.25) (layer "F.Cu") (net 16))
 (segment (start 259.35 47.1625) (end 259.35 53.12) (width 0.25) (layer "F.Cu") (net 16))
 (segment (start 257.575 72.625) (end 267.1 82.15) (width 2) (layer "F.Cu") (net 16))
 (segment (start 259.35 74.4) (end 267.1 82.15) (width 0.25) (layer "F.Cu") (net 16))
 (segment (start 259.35 53.12) (end 257.575 54.895) (width 0.25) (layer "F.Cu") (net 16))
 (segment (start 260.2375 82) (end 266.95 82) (width 1) (layer "F.Cu") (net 16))
 (segment (start 257.575 58.705) (end 257.575 72.625) (width 2) (layer "F.Cu") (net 16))
 (segment (start 262.63 48.115) (end 260.3025 48.115) (width 0.25) (layer "F.Cu") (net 16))
 (segment (start 257.575 56.165) (end 257.575 58.705) (width 2) (layer "F.Cu") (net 16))
 (segment (start 266.95 82) (end 267.1 82.15) (width 1) (layer "F.Cu") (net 16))
 (segment (start 257.575 56.165) (end 257.575 54.895) (width 2) (layer "F.Cu") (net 16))
 (segment (start 246.325 52.959) (end 246.325 49.149) (width 2) (layer "F.Cu") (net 19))
 (segment (start 254.508 54.102) (end 254.508 57.912) (width 0.25) (layer "F.Cu") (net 12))
 (segment (start 257.048 43.213569) (end 257.048 51.562) (width 0.25) (layer "F.Cu") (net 12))
 (segment (start 254.508 57.912) (end 253.715 58.705) (width 0.25) (layer "F.Cu") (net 12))
 (segment (start 257.048 51.562) (end 254.508 54.102) (width 0.25) (layer "F.Cu") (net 12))
 (segment (start 254.901931 41.0675) (end 257.048 43.213569) (width 0.25) (layer "F.Cu") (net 12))
 (segment (start 254.065 41.0675) (end 254.901931 41.0675) (width 0.25) (layer "F.Cu") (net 12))
 (segment (start 253.715 58.705) (end 252.625 58.705) (width 0.25) (layer "F.Cu") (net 12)))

